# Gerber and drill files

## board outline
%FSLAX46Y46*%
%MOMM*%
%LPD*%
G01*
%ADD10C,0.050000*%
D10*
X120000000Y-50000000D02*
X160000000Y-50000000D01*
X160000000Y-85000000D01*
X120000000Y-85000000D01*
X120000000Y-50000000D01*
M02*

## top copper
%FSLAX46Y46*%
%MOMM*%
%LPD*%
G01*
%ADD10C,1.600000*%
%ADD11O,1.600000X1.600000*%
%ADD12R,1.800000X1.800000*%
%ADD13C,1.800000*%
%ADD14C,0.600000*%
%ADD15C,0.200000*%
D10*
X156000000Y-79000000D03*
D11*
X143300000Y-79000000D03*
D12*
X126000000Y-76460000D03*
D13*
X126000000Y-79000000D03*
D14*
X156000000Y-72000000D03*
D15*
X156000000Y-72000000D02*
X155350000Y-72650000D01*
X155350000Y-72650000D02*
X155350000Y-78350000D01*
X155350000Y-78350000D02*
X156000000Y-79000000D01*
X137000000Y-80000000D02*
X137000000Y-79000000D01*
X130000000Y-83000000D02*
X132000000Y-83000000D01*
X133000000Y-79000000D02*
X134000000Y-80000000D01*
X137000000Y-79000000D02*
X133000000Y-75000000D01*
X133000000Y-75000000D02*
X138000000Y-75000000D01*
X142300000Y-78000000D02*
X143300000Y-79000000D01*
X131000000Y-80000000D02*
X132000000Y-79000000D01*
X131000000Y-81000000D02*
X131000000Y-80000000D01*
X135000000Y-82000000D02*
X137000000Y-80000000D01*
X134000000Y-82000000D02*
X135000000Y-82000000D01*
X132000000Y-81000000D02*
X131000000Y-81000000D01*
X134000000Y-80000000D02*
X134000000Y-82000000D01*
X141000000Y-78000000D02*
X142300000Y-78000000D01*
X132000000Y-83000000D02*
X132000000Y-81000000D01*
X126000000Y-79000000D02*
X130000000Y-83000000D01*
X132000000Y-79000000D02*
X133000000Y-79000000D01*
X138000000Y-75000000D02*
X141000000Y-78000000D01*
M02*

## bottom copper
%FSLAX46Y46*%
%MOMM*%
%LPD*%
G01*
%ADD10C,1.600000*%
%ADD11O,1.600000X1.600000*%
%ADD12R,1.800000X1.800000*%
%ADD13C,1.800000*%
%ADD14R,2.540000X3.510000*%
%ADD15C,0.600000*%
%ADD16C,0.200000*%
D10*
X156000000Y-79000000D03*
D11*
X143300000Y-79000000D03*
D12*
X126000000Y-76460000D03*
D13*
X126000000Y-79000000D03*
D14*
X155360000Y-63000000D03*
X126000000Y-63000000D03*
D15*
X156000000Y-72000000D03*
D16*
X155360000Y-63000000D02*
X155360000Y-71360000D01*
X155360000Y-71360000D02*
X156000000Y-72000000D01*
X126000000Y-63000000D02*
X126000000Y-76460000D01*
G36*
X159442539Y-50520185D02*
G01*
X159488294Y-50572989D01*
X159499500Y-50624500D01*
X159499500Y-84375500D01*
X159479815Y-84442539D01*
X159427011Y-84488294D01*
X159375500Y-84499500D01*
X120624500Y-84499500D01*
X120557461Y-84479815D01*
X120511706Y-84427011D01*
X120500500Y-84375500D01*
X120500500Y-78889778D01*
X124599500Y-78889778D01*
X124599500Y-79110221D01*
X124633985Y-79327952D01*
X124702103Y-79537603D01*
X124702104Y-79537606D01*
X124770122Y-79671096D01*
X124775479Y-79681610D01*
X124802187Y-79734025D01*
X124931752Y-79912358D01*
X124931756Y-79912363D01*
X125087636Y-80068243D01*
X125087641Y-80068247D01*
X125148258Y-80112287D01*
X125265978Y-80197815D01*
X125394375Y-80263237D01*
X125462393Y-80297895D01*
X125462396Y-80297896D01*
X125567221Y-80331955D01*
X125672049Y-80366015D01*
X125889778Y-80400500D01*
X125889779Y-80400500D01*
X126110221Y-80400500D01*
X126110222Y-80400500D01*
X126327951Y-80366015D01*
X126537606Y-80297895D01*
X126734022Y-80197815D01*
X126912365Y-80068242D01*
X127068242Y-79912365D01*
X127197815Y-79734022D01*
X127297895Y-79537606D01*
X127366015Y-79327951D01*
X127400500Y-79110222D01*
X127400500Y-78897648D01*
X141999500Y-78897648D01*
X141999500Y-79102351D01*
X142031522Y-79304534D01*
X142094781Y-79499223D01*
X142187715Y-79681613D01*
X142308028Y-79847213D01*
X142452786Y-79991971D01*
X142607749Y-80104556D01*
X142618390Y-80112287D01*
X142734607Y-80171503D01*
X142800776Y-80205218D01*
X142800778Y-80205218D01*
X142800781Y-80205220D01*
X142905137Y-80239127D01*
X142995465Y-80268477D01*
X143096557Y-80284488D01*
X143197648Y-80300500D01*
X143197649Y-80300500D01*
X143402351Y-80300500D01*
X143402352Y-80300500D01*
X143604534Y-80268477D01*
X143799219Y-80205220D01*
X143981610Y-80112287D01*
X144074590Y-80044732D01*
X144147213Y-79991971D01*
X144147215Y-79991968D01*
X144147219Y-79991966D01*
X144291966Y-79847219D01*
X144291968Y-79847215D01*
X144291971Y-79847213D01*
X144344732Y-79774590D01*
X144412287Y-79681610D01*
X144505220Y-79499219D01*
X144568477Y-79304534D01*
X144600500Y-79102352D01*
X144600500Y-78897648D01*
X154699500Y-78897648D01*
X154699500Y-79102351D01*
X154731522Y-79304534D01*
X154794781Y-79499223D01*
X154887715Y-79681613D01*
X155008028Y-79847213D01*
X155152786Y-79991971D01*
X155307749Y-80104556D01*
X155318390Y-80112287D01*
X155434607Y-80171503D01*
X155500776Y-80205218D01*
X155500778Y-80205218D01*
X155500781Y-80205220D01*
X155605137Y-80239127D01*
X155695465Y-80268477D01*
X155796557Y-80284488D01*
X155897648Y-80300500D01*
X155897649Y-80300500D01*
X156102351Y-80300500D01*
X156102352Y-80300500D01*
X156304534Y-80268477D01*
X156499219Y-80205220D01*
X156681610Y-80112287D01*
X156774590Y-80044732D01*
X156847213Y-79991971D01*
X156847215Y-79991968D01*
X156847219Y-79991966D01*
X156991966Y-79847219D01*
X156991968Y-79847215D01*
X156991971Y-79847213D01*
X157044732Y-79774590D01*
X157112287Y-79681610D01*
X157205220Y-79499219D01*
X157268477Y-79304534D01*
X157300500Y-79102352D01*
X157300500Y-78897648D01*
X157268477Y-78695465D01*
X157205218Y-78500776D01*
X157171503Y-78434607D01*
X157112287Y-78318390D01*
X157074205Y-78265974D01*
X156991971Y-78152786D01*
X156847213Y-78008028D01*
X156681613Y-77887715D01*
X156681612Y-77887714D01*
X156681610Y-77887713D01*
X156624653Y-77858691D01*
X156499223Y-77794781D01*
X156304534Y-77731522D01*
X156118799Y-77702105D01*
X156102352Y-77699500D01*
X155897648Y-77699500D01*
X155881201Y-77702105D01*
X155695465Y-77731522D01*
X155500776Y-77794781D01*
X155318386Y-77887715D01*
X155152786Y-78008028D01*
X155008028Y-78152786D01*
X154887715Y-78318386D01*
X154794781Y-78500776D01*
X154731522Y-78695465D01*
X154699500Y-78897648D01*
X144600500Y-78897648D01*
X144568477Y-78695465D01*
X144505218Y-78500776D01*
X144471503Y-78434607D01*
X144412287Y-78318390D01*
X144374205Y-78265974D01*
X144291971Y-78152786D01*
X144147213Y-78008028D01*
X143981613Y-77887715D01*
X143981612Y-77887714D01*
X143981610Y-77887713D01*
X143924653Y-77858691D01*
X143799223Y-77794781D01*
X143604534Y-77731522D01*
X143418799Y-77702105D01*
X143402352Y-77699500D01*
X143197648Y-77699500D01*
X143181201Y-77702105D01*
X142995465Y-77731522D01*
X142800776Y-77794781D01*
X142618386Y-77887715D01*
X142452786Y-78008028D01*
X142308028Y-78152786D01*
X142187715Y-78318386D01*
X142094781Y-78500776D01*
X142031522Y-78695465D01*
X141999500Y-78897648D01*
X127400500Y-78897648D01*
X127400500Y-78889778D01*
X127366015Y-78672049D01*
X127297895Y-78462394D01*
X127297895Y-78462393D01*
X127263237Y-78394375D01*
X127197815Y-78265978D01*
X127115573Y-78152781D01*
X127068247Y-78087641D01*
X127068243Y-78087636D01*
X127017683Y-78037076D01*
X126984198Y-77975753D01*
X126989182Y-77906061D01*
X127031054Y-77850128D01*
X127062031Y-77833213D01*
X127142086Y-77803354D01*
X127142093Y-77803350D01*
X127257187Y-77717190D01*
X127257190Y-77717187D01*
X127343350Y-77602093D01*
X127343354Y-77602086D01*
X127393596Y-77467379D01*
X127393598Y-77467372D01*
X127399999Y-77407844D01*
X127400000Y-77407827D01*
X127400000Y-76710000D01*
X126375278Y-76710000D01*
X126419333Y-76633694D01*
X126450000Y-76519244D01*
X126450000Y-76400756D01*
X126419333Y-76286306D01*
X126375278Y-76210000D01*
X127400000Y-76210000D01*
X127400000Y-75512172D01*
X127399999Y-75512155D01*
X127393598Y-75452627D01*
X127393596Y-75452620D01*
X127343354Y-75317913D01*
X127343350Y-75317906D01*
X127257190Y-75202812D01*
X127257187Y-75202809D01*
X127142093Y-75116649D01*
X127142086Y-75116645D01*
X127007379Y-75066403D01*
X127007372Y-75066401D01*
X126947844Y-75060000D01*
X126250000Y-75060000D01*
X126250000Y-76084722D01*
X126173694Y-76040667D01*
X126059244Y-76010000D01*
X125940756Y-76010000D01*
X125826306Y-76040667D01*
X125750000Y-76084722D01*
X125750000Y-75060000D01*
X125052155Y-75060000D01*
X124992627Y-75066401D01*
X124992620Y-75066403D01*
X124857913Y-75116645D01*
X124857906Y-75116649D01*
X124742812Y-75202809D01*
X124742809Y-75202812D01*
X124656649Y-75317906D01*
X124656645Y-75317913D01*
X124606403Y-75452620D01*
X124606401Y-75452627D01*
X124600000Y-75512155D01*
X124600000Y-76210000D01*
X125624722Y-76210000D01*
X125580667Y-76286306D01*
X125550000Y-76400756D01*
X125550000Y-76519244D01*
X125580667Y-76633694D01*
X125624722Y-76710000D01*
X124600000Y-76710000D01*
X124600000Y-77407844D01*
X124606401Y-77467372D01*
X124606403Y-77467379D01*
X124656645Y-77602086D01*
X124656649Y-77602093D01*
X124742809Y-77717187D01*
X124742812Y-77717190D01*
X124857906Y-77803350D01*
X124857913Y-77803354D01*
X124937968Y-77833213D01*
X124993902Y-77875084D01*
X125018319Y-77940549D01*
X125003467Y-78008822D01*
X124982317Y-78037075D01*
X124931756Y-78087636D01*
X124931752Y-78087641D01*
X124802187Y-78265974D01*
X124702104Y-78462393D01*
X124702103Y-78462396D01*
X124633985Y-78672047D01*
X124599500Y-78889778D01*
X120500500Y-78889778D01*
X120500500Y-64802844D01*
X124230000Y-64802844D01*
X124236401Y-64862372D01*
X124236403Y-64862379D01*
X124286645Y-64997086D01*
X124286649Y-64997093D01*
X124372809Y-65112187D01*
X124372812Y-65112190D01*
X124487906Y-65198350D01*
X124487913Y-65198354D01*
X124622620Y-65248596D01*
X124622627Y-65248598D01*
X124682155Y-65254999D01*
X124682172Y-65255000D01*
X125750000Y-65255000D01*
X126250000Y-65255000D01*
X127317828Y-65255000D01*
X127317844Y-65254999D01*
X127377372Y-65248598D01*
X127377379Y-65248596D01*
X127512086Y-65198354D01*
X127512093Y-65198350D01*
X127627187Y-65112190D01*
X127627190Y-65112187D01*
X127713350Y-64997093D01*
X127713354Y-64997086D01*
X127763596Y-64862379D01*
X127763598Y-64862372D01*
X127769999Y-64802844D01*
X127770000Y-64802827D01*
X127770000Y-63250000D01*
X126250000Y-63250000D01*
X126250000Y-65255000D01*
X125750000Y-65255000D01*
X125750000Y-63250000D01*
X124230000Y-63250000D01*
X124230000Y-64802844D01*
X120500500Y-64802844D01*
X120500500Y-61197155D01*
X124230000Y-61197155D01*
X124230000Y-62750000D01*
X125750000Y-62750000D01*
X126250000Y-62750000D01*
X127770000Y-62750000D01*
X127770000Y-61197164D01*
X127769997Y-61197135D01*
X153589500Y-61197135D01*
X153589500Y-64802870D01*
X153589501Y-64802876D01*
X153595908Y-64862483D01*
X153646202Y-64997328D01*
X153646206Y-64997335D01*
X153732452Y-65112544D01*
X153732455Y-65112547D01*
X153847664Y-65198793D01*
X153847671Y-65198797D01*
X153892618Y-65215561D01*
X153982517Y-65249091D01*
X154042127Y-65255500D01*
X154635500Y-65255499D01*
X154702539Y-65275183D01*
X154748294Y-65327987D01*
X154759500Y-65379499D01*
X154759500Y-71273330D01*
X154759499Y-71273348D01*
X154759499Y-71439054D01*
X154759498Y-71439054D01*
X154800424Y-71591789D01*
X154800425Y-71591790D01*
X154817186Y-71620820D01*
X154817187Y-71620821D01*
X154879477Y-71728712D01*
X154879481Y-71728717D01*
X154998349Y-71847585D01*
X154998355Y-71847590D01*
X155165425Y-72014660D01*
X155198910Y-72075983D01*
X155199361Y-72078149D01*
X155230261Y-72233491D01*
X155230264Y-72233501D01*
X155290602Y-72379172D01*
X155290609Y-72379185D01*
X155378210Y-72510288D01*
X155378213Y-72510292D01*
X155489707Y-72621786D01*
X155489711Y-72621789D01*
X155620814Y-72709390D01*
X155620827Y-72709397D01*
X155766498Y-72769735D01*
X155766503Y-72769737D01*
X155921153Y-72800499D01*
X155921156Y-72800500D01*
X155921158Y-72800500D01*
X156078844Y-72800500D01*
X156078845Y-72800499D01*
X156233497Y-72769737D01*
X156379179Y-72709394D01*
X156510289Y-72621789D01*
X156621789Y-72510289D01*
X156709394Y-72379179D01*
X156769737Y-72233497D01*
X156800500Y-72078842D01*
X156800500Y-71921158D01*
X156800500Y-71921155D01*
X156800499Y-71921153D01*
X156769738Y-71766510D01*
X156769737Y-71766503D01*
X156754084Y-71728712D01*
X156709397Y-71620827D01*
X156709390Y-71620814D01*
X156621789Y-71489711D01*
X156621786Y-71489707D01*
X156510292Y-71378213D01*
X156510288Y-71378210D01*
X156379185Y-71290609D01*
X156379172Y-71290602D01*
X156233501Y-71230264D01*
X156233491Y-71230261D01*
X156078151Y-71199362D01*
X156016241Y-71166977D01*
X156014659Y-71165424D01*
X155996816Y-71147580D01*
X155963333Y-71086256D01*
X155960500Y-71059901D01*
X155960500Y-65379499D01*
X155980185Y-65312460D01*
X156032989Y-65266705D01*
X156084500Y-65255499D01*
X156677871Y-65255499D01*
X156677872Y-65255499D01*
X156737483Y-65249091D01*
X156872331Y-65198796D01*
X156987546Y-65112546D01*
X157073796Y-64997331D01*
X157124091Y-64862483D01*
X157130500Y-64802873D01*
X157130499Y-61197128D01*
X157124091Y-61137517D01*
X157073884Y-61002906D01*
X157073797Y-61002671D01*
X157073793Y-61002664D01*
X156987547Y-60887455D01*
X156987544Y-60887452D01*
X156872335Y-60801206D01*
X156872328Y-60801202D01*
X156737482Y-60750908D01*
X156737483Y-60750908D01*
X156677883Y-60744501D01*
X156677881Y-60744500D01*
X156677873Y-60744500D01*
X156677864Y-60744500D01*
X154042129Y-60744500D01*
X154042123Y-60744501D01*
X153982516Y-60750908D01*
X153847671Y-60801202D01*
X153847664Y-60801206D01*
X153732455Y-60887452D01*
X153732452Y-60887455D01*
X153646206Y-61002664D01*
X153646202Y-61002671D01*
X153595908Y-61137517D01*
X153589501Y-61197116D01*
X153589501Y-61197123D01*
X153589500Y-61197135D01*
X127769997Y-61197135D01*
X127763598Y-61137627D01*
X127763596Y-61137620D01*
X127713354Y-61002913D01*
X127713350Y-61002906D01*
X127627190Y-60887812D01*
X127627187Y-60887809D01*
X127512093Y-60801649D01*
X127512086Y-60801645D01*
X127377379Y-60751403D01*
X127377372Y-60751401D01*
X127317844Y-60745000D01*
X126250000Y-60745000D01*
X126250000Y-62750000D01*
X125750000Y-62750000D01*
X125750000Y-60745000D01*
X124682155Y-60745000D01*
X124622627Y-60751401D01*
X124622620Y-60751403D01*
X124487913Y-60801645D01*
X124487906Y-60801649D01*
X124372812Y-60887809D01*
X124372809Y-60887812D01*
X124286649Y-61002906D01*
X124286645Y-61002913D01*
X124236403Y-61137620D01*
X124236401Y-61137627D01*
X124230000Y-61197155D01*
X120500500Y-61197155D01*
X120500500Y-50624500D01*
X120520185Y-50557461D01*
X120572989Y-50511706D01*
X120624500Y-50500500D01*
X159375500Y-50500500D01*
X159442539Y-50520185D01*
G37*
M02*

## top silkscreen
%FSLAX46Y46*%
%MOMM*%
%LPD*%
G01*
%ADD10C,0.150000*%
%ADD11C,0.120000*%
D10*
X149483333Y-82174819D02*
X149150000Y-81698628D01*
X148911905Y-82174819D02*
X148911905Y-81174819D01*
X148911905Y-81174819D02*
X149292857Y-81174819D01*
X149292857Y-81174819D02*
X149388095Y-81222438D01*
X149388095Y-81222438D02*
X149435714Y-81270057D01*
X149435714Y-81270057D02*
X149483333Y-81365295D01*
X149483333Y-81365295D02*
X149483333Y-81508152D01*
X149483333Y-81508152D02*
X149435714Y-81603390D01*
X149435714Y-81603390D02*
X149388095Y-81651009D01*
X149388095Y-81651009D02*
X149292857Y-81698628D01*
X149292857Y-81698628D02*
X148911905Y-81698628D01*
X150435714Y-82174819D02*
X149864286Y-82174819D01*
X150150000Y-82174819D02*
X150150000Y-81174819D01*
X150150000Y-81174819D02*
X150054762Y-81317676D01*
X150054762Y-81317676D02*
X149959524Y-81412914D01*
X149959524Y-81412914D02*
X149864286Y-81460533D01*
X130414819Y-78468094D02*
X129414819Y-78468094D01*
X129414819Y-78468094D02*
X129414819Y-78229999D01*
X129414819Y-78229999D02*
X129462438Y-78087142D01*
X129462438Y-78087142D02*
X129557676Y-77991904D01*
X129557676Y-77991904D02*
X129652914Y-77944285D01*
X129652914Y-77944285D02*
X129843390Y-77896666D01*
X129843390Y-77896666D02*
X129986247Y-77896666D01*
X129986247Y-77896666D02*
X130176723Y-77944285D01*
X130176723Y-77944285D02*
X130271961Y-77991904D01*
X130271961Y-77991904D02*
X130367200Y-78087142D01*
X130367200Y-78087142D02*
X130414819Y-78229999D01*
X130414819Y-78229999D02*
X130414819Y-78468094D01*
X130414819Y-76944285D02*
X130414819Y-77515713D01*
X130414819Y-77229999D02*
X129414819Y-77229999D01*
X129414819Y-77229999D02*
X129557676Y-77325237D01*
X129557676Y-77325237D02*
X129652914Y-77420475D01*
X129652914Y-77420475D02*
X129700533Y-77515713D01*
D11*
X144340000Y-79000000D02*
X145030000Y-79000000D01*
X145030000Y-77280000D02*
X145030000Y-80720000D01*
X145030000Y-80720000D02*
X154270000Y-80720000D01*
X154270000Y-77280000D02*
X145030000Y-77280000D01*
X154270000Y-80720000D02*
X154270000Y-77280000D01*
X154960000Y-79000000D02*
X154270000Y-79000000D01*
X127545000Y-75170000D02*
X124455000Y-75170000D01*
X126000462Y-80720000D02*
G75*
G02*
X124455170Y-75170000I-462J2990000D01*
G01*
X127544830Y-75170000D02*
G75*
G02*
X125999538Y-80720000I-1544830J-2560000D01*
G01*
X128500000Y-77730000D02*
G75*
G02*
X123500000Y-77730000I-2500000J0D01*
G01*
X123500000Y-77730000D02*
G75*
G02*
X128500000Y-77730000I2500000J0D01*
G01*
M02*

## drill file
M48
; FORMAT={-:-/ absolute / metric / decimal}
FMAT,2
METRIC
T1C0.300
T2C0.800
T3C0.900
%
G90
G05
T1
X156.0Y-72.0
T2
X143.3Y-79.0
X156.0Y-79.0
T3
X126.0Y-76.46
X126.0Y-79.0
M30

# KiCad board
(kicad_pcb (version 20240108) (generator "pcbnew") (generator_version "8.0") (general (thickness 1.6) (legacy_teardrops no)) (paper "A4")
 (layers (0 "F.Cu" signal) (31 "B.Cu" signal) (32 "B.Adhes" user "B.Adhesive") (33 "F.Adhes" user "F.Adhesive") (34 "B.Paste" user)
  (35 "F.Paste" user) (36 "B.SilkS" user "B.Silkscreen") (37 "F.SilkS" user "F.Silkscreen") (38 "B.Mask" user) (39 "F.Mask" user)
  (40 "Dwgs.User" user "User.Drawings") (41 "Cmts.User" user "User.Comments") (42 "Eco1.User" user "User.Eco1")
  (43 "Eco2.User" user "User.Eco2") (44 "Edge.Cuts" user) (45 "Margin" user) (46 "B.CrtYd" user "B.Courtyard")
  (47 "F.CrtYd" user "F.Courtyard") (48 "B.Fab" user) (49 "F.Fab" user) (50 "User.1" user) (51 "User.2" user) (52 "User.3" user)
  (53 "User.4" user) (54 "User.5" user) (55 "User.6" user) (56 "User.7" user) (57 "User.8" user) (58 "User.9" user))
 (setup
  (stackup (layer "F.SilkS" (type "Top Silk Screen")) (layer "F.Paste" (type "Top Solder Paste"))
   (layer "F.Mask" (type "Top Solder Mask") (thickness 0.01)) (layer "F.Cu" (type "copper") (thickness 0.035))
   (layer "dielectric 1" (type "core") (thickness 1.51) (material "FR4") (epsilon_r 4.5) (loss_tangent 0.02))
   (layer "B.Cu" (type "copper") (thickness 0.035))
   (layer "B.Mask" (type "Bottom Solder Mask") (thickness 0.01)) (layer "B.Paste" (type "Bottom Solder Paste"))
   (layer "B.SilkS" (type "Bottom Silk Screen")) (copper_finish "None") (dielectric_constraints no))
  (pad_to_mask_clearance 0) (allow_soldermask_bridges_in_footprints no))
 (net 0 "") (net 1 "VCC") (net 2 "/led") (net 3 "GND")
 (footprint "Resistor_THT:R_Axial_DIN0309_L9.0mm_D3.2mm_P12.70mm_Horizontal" (layer "F.Cu") (at 156 79 180)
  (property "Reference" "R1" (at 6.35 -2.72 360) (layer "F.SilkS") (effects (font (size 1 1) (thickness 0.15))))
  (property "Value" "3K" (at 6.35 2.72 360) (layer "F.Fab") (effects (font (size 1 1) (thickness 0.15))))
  (fp_line (start 11.66 0) (end 10.97 0) (stroke (width 0.12) (type solid)) (layer "F.SilkS"))
  (fp_line (start 10.97 1.72) (end 10.97 -1.72) (stroke (width 0.12) (type solid)) (layer "F.SilkS"))
  (fp_line (start 10.97 -1.72) (end 1.73 -1.72) (stroke (width 0.12) (type solid)) (layer "F.SilkS"))
  (fp_line (start 1.73 1.72) (end 10.97 1.72) (stroke (width 0.12) (type solid)) (layer "F.SilkS"))
  (fp_line (start 1.73 -1.72) (end 1.73 1.72) (stroke (width 0.12) (type solid)) (layer "F.SilkS"))
  (fp_line (start 1.04 0) (end 1.73 0) (stroke (width 0.12) (type solid)) (layer "F.SilkS"))
  (pad "1" thru_hole circle (at 0 0 180) (size 1.6 1.6) (drill 0.8) (layers "*.Cu" "*.Mask") (remove_unused_layers no) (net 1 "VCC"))
  (pad "2" thru_hole oval (at 12.7 0 180) (size 1.6 1.6) (drill 0.8) (layers "*.Cu" "*.Mask") (remove_unused_layers no) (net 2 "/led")))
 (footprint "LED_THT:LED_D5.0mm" (layer "F.Cu") (at 126 76.46 -90)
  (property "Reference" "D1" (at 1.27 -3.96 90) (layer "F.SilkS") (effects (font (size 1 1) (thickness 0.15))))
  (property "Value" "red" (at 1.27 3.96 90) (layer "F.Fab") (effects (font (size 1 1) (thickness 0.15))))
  (fp_line (start -1.29 -1.545) (end -1.29 1.545) (stroke (width 0.12) (type solid)) (layer "F.SilkS"))
  (fp_arc (start 4.26 -0.000462) (mid 2.072002 2.880433) (end -1.29 1.54483) (stroke (width 0.12) (type solid)) (layer "F.SilkS"))
  (fp_arc (start -1.29 -1.54483) (mid 2.072002 -2.880433) (end 4.26 0.000462) (stroke (width 0.12) (type solid)) (layer "F.SilkS"))
  (fp_circle (center 1.27 0) (end 3.77 0) (stroke (width 0.12) (type solid)) (fill none) (layer "F.SilkS"))
  (pad "1" thru_hole rect (at 0 0 270) (size 1.8 1.8) (drill 0.9) (layers "*.Cu" "*.Mask") (remove_unused_layers no) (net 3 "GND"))
  (pad "2" thru_hole circle (at 2.54 0 270) (size 1.8 1.8) (drill 0.9) (layers "*.Cu" "*.Mask") (remove_unused_layers no) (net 2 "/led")))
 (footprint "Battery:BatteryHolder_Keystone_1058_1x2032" (layer "B.Cu") (at 140.68 63 180)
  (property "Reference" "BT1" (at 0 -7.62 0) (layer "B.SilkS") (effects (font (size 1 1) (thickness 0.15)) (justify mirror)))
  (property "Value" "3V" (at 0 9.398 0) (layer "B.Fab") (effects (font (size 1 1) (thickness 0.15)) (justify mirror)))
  (pad "1" smd rect (at -14.68 0 180) (size 2.54 3.51) (layers "B.Cu" "B.Paste" "B.Mask") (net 1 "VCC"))
  (pad "2" smd rect (at 14.68 0 180) (size 2.54 3.51) (layers "B.Cu" "B.Paste" "B.Mask") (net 3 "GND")))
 (gr_rect (start 120 50) (end 160 85) (stroke (width 0.05) (type default)) (fill none) (layer "Edge.Cuts"))
 (segment (start 156 72) (end 155.35 72.65) (width 0.2) (layer "F.Cu") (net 1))
 (segment (start 155.35 72.65) (end 155.35 78.35) (width 0.2) (layer "F.Cu") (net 1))
 (segment (start 155.35 78.35) (end 156 79) (width 0.2) (layer "F.Cu") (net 1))
 (via (at 156 72) (size 0.6) (drill 0.3) (layers "F.Cu" "B.Cu") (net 1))
 (segment (start 155.36 63) (end 155.36 71.36) (width 0.2) (layer "B.Cu") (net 1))
 (segment (start 155.36 71.36) (end 156 72) (width 0.2) (layer "B.Cu") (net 1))
 (segment (start 126 63) (end 126 76.46) (width 0.2) (layer "B.Cu") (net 3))
 (segment (start 137 80) (end 137 79) (width 0.2) (layer "F.Cu") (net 2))
 (segment (start 130 83) (end 132 83) (width 0.2) (layer "F.Cu") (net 2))
 (segment (start 133 79) (end 134 80) (width 0.2) (layer "F.Cu") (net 2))
 (segment (start 137 79) (end 133 75) (width 0.2) (layer "F.Cu") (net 2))
 (segment (start 133 75) (end 138 75) (width 0.2) (layer "F.Cu") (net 2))
 (segment (start 142.3 78) (end 143.3 79) (width 0.2) (layer "F.Cu") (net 2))
 (segment (start 131 80) (end 132 79) (width 0.2) (layer "F.Cu") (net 2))
 (segment (start 131 81) (end 131 80) (width 0.2) (layer "F.Cu") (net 2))
 (segment (start 135 82) (end 137 80) (width 0.2) (layer "F.Cu") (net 2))
 (segment (start 134 82) (end 135 82) (width 0.2) (layer "F.Cu") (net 2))
 (segment (start 132 81) (end 131 81) (width 0.2) (layer "F.Cu") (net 2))
 (segment (start 134 80) (end 134 82) (width 0.2) (layer "F.Cu") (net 2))
 (segment (start 141 78) (end 142.3 78) (width 0.2) (layer "F.Cu") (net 2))
 (segment (start 132 83) (end 132 81) (width 0.2) (layer "F.Cu") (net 2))
 (segment (start 126 79) (end 130 83) (width 0.2) (layer "F.Cu") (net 2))
 (segment (start 132 79) (end 133 79) (width 0.2) (layer "F.Cu") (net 2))
 (segment (start 138 75) (end 141 78) (width 0.2) (layer "F.Cu") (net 2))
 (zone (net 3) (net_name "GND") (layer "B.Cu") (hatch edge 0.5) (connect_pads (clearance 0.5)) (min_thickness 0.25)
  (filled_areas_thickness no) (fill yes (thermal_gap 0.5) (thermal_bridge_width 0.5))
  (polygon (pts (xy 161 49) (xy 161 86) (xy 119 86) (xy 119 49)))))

